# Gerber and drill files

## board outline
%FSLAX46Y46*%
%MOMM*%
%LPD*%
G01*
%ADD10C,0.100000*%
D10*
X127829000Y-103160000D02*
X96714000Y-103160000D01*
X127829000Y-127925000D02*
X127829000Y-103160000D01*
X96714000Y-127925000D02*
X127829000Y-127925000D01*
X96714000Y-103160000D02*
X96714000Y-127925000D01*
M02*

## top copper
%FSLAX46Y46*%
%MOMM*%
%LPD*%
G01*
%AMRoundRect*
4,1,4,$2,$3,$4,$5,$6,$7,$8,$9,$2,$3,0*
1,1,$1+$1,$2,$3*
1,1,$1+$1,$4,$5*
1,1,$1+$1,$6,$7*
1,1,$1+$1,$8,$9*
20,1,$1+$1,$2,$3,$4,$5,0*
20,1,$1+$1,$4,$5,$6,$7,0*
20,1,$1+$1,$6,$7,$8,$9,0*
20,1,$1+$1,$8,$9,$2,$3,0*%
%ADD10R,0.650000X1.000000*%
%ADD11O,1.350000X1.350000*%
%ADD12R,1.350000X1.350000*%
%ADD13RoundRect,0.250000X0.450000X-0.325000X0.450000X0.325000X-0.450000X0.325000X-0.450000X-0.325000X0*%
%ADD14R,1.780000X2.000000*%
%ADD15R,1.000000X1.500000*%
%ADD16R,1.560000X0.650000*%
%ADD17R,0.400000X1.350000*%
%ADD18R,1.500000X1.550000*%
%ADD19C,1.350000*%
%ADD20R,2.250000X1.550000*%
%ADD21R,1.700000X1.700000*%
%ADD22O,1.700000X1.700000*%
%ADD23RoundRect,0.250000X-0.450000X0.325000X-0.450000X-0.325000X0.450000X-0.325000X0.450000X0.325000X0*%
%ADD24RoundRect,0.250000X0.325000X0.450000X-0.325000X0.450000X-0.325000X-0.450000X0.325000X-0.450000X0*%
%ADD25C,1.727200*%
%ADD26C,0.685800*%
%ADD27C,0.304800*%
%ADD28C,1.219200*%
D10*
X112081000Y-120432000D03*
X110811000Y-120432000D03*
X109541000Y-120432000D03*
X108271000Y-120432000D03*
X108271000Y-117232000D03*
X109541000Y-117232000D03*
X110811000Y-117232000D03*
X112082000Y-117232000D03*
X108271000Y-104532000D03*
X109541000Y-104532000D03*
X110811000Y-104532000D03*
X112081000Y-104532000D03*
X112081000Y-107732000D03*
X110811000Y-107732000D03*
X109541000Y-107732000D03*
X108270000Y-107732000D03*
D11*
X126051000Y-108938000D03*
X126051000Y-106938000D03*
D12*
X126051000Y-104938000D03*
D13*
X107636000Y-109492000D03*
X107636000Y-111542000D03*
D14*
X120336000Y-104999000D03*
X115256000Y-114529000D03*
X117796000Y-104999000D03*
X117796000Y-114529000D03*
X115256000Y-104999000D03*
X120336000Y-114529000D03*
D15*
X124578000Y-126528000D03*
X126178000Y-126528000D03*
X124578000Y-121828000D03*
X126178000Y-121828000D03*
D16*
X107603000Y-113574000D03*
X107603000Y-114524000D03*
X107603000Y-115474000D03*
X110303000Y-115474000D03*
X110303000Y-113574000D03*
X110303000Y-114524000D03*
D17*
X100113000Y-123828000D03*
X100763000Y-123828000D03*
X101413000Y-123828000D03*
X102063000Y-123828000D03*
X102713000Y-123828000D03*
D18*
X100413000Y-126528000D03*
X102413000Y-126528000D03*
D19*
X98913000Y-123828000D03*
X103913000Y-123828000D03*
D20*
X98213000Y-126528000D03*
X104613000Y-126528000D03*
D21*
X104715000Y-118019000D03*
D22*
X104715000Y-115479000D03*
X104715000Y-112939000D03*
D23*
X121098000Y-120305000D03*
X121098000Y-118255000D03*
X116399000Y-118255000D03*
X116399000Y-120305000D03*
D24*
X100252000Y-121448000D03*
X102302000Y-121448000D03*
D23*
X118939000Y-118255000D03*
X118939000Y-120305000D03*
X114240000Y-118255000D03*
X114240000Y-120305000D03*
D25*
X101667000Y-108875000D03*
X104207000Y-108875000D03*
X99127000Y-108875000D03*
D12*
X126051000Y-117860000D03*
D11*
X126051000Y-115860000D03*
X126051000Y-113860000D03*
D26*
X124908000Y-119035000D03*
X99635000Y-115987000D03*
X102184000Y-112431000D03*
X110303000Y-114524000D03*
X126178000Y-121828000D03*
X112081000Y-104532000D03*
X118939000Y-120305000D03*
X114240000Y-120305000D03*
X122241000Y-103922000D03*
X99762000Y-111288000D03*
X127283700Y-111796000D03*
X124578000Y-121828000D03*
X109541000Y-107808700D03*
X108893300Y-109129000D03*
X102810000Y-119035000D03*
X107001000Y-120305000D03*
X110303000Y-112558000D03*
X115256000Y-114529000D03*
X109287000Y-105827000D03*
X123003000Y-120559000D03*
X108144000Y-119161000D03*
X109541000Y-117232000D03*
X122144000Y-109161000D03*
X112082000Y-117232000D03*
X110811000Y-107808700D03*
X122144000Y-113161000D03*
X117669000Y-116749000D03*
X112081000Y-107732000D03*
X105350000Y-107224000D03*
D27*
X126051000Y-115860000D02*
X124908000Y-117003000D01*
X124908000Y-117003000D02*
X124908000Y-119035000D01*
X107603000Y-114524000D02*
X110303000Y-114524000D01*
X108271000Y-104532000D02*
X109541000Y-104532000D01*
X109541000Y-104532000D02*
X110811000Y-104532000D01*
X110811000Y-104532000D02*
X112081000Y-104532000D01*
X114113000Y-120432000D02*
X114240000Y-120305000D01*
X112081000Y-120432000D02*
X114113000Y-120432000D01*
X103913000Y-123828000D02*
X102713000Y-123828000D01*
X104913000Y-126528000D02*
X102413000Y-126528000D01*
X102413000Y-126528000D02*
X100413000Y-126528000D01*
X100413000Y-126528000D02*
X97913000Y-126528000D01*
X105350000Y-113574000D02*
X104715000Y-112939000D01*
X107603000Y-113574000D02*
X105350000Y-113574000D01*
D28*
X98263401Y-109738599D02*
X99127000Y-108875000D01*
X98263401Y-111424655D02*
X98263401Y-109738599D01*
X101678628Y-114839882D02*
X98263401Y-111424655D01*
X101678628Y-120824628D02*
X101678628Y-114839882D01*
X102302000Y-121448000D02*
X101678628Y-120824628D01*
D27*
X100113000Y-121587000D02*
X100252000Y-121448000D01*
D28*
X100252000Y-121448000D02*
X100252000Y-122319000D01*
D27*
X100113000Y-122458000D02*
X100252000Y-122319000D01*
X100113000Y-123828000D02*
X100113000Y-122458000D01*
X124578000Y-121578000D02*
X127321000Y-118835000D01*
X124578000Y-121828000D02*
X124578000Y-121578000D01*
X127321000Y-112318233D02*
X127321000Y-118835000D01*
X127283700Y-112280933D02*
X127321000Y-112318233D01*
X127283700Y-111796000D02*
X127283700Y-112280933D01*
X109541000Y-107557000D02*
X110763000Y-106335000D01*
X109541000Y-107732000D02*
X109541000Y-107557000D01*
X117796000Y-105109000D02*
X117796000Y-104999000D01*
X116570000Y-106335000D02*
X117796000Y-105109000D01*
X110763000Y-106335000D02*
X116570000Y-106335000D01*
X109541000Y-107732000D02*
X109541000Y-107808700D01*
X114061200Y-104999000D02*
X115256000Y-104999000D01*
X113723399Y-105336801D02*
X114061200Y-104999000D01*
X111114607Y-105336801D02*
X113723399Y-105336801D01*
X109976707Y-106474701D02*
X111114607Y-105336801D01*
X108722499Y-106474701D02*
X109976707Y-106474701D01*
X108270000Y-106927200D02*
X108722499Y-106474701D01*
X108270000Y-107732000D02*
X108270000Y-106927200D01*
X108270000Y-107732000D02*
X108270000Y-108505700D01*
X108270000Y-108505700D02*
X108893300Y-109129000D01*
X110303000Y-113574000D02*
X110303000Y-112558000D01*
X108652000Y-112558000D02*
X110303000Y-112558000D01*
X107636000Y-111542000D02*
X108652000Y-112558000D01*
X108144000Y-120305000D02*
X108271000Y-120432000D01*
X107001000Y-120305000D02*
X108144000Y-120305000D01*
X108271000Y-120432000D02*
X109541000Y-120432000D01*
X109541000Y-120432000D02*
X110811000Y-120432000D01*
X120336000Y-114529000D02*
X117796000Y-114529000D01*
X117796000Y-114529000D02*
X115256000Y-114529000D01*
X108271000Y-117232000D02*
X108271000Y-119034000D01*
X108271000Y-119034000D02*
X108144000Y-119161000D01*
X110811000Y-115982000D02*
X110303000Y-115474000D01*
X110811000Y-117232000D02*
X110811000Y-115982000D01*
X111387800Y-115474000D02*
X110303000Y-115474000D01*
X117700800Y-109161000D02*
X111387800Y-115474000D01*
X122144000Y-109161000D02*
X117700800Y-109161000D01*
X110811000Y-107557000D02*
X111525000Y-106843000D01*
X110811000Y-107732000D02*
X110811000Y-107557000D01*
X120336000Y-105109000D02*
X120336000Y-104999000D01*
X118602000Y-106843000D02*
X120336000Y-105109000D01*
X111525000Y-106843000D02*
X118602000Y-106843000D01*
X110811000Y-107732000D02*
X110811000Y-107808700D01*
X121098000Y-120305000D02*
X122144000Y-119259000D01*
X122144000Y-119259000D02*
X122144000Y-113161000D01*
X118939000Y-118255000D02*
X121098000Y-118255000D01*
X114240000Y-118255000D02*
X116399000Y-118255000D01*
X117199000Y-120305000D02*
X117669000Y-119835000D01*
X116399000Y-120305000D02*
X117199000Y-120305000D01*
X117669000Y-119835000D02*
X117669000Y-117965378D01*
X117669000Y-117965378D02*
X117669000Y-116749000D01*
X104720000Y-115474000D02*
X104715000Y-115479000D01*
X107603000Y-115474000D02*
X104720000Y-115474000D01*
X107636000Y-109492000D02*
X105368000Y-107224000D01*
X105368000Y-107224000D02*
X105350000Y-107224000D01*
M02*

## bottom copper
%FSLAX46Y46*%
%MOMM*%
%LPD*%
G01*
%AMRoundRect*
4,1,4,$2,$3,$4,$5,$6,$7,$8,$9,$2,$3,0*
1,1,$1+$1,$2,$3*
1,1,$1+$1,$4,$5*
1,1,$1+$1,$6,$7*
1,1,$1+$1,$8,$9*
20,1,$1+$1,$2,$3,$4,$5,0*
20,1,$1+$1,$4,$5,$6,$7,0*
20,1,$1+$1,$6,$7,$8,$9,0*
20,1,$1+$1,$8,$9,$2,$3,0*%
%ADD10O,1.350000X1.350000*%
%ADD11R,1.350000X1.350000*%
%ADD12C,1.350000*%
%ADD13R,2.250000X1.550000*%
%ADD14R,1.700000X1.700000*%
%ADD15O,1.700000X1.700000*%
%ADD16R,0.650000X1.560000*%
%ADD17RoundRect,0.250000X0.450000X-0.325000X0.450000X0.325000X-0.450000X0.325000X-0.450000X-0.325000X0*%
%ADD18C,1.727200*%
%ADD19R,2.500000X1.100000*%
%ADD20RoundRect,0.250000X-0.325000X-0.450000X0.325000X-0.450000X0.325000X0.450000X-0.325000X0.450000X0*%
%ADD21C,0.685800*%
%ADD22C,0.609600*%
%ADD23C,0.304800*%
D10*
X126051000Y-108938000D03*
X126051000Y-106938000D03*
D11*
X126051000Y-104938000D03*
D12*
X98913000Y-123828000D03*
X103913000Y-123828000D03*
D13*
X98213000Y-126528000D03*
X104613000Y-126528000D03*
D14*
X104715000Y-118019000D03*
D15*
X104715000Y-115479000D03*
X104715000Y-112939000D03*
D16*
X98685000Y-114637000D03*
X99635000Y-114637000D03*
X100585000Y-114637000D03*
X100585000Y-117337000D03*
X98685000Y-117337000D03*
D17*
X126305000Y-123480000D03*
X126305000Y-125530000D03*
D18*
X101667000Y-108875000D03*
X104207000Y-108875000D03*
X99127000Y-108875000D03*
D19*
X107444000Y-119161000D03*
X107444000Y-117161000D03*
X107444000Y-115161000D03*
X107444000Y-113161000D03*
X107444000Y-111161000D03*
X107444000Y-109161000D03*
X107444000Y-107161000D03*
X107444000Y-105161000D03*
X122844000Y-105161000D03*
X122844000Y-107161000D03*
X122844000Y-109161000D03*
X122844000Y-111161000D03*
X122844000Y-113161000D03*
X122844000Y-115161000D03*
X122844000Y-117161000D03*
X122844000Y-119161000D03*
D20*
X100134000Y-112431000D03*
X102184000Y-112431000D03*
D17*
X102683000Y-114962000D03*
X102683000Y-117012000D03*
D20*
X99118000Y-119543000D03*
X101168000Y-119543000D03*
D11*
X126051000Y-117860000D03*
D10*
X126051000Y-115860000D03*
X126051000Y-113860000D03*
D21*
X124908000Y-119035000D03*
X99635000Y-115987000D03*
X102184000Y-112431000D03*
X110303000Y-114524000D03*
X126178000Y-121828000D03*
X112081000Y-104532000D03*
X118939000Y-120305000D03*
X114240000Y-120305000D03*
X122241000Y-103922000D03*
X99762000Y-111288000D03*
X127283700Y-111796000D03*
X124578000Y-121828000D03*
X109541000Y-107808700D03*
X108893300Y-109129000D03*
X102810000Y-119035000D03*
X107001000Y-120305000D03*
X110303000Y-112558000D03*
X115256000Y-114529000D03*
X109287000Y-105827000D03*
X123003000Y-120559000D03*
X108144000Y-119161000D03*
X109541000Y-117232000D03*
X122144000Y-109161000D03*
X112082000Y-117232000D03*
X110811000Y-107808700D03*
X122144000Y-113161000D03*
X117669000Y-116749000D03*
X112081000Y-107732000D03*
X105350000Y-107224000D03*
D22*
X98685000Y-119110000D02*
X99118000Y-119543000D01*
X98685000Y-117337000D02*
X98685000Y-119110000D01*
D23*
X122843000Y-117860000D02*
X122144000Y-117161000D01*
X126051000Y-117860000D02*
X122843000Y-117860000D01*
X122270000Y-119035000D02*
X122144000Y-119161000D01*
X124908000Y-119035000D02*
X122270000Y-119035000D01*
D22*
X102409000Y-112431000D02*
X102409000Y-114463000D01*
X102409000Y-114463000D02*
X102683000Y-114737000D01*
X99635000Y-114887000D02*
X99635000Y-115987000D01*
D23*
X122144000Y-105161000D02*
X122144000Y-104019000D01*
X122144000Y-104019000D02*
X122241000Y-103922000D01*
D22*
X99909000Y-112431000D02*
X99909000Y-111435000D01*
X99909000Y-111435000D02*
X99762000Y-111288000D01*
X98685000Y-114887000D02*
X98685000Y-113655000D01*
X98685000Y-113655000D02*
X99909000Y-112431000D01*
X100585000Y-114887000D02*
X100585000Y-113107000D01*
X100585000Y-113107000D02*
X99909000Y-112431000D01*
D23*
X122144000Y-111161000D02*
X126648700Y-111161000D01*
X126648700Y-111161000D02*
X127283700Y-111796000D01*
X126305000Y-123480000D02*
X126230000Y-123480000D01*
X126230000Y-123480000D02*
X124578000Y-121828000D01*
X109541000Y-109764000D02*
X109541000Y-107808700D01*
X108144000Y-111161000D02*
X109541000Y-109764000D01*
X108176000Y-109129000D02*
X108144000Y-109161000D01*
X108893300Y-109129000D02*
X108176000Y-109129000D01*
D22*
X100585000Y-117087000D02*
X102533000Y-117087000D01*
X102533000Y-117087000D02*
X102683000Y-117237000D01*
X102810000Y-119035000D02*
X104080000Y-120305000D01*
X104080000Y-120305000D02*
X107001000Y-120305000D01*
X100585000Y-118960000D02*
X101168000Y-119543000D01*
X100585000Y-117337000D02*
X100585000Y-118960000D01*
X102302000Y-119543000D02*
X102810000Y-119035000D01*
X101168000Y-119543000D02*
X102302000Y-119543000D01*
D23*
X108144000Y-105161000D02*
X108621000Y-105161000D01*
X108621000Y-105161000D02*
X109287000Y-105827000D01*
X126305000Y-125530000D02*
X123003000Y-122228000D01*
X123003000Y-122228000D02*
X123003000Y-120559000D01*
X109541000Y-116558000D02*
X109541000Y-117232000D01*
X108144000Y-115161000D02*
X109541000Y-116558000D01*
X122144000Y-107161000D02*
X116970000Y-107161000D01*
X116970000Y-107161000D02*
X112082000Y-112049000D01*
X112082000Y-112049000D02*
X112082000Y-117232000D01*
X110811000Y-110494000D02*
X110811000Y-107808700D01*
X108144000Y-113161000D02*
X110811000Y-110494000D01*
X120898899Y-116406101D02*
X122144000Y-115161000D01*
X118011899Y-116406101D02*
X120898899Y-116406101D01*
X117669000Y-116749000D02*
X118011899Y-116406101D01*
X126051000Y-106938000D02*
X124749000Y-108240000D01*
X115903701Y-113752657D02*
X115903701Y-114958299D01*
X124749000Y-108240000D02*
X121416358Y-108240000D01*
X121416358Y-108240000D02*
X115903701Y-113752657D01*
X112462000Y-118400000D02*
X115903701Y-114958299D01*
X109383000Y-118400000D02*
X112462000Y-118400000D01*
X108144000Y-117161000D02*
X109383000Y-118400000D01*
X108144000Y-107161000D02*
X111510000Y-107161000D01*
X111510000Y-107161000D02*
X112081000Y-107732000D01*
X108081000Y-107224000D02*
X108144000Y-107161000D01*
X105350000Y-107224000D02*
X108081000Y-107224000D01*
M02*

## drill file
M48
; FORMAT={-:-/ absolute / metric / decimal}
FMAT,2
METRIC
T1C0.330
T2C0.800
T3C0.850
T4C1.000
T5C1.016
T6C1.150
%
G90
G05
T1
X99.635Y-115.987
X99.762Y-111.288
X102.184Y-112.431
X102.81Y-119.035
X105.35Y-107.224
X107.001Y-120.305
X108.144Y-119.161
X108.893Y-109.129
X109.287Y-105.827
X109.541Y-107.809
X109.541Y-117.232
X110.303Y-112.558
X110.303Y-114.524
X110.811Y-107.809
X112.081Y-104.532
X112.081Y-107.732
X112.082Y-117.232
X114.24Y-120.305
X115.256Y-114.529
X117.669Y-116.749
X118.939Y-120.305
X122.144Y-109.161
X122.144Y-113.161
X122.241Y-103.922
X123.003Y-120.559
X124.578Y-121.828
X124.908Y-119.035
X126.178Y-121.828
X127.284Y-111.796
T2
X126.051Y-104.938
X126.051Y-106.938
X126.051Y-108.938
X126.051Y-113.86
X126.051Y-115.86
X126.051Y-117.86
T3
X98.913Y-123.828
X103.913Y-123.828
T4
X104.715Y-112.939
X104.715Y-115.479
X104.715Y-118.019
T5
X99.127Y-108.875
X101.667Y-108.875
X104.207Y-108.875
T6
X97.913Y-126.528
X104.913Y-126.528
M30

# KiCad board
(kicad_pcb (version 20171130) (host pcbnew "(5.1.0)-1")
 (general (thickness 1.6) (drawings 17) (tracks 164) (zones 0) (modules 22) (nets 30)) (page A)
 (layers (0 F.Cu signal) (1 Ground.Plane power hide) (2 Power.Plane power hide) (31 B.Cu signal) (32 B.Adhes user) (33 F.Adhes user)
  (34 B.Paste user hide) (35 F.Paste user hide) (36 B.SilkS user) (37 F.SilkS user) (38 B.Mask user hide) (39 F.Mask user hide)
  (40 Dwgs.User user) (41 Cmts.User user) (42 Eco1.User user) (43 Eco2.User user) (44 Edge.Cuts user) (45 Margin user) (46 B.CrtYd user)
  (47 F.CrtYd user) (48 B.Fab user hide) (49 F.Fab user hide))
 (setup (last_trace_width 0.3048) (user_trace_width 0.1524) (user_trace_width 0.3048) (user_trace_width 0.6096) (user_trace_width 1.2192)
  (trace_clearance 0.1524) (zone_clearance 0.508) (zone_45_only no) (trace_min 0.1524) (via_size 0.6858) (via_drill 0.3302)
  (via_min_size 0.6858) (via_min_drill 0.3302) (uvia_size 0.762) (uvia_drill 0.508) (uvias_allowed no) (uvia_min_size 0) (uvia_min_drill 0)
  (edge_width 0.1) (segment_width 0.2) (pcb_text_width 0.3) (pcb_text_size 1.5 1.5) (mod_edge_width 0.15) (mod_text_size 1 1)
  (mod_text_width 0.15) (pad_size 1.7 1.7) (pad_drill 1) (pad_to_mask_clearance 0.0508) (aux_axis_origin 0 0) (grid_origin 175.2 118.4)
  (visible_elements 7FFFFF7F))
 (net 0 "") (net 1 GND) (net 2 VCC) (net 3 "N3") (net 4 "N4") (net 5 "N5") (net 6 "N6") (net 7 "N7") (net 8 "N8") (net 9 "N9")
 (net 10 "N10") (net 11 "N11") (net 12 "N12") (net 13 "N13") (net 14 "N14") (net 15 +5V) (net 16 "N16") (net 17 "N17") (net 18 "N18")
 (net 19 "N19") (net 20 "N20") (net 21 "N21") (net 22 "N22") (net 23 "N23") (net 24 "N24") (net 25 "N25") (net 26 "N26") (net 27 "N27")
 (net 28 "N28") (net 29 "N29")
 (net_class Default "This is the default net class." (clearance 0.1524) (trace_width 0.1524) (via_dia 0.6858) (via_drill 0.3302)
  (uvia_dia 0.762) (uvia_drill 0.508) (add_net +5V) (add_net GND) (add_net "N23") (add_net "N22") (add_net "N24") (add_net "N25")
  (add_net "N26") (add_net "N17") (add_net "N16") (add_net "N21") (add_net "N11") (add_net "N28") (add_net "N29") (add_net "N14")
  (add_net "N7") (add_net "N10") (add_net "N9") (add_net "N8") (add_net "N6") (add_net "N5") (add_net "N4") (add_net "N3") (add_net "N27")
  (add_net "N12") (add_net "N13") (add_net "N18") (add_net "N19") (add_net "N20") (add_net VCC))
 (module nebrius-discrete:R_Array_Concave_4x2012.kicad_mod (layer F.Cu) (at 110.176 118.832 180)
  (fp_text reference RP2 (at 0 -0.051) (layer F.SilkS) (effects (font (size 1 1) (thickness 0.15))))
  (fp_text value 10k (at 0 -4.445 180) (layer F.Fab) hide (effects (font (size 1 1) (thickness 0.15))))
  (pad 8 smd rect (at -1.905 -1.6 180) (size 0.65 1) (layers F.Cu F.Paste F.Mask) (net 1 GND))
  (pad 7 smd rect (at -0.635 -1.6 180) (size 0.65 1) (layers F.Cu F.Paste F.Mask) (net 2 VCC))
  (pad 6 smd rect (at 0.635 -1.6 180) (size 0.65 1) (layers F.Cu F.Paste F.Mask) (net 2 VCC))
  (pad 5 smd rect (at 1.905 -1.6 180) (size 0.65 1) (layers F.Cu F.Paste F.Mask) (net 2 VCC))
  (pad 4 smd rect (at 1.905 1.6 180) (size 0.65 1) (layers F.Cu F.Paste F.Mask) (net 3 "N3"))
  (pad 3 smd rect (at 0.635 1.6 180) (size 0.65 1) (layers F.Cu F.Paste F.Mask) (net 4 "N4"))
  (pad 2 smd rect (at -0.635 1.6 180) (size 0.65 1) (layers F.Cu F.Paste F.Mask) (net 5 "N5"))
  (pad 1 smd rect (at -1.906 1.6 180) (size 0.65 1) (layers F.Cu F.Paste F.Mask) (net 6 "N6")))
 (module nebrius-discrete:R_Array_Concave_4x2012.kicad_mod (layer F.Cu) (at 110.176 106.132)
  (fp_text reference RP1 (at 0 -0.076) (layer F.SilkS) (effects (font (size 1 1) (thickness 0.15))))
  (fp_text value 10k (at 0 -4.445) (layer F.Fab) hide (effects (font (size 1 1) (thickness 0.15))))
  (pad 8 smd rect (at -1.905 -1.6) (size 0.65 1) (layers F.Cu F.Paste F.Mask) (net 1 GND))
  (pad 7 smd rect (at -0.635 -1.6) (size 0.65 1) (layers F.Cu F.Paste F.Mask) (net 1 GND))
  (pad 6 smd rect (at 0.635 -1.6) (size 0.65 1) (layers F.Cu F.Paste F.Mask) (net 1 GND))
  (pad 5 smd rect (at 1.905 -1.6) (size 0.65 1) (layers F.Cu F.Paste F.Mask) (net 1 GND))
  (pad 4 smd rect (at 1.905 1.6) (size 0.65 1) (layers F.Cu F.Paste F.Mask) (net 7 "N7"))
  (pad 3 smd rect (at 0.635 1.6) (size 0.65 1) (layers F.Cu F.Paste F.Mask) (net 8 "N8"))
  (pad 2 smd rect (at -0.635 1.6) (size 0.65 1) (layers F.Cu F.Paste F.Mask) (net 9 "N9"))
  (pad 1 smd rect (at -1.906 1.6) (size 0.65 1) (layers F.Cu F.Paste F.Mask) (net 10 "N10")))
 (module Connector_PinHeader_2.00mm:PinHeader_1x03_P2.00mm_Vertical (layer F.Cu) (at 126.051 104.938)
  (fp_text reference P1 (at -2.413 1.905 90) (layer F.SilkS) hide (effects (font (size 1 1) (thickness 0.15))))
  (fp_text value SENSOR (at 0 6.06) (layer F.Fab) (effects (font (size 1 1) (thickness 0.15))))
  (pad 3 thru_hole oval (at 0 4) (size 1.35 1.35) (drill 0.8) (layers *.Cu *.Mask) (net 1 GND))
  (pad 2 thru_hole oval (at 0 2) (size 1.35 1.35) (drill 0.8) (layers *.Cu *.Mask) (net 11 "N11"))
  (pad 1 thru_hole rect (at 0 0) (size 1.35 1.35) (drill 0.8) (layers *.Cu *.Mask) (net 2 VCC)))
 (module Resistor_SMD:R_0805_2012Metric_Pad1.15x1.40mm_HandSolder (layer F.Cu) (at 107.636 110.517 90)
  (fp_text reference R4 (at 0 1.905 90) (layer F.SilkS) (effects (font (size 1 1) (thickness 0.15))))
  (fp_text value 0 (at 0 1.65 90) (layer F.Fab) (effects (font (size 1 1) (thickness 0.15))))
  (pad 2 smd roundrect (at 1.025 0 90) (size 1.15 1.4) (layers F.Cu F.Paste F.Mask) (roundrect_rratio 0.217391) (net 7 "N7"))
  (pad 1 smd roundrect (at -1.025 0 90) (size 1.15 1.4) (layers F.Cu F.Paste F.Mask) (roundrect_rratio 0.217391) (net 2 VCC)))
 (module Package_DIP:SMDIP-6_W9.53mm (layer F.Cu) (at 117.796 109.764 270)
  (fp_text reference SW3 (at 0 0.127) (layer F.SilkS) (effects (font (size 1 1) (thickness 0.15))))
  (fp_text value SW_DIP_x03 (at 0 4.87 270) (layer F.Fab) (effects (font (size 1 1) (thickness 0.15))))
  (pad 1 smd rect (at -4.765 -2.54 270) (size 2 1.78) (layers F.Cu F.Paste F.Mask) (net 8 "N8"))
  (pad 4 smd rect (at 4.765 2.54 270) (size 2 1.78) (layers F.Cu F.Paste F.Mask) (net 2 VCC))
  (pad 2 smd rect (at -4.765 0 270) (size 2 1.78) (layers F.Cu F.Paste F.Mask) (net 9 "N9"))
  (pad 5 smd rect (at 4.765 0 270) (size 2 1.78) (layers F.Cu F.Paste F.Mask) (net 2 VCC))
  (pad 3 smd rect (at -4.765 2.54 270) (size 2 1.78) (layers F.Cu F.Paste F.Mask) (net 10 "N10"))
  (pad 6 smd rect (at 4.765 -2.54 270) (size 2 1.78) (layers F.Cu F.Paste F.Mask) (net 2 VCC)))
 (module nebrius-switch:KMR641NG (layer F.Cu) (at 125.378 124.178 90)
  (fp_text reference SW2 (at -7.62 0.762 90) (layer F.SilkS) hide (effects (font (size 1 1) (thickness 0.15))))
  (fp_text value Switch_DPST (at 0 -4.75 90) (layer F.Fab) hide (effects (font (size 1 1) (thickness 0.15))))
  (pad 1 smd rect (at -2.35 -0.8 90) (size 1.5 1) (layers F.Cu F.Paste F.Mask) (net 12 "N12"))
  (pad 2 smd rect (at -2.35 0.8 90) (size 1.5 1) (layers F.Cu F.Paste F.Mask) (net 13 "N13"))
  (pad 3 smd rect (at 2.35 -0.8 90) (size 1.5 1) (layers F.Cu F.Paste F.Mask) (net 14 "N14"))
  (pad 4 smd rect (at 2.35 0.8 90) (size 1.5 1) (layers F.Cu F.Paste F.Mask) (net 1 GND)))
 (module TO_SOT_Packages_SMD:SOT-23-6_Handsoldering (layer F.Cu) (at 108.953 114.524)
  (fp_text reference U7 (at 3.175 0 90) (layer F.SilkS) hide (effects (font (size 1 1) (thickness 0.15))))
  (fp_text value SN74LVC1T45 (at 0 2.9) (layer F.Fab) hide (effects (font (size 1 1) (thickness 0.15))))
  (pad 1 smd rect (at -1.35 -0.95) (size 1.56 0.65) (layers F.Cu F.Paste F.Mask) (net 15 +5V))
  (pad 2 smd rect (at -1.35 0) (size 1.56 0.65) (layers F.Cu F.Paste F.Mask) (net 1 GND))
  (pad 3 smd rect (at -1.35 0.95) (size 1.56 0.65) (layers F.Cu F.Paste F.Mask) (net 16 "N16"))
  (pad 4 smd rect (at 1.35 0.95) (size 1.56 0.65) (layers F.Cu F.Paste F.Mask) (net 5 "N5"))
  (pad 6 smd rect (at 1.35 -0.95) (size 1.56 0.65) (layers F.Cu F.Paste F.Mask) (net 2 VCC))
  (pad 5 smd rect (at 1.35 0) (size 1.56 0.65) (layers F.Cu F.Paste F.Mask) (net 1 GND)))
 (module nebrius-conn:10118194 (layer F.Cu) (at 101.413 126.528)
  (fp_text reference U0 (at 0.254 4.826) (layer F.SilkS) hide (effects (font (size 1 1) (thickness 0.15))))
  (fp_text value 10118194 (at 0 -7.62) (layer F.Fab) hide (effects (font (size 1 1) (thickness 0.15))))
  (pad 1 smd rect (at -1.3 -2.7) (size 0.4 1.35) (layers F.Cu F.Paste F.Mask) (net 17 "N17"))
  (pad 2 smd rect (at -0.65 -2.7) (size 0.4 1.35) (layers F.Cu F.Paste F.Mask) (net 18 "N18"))
  (pad 3 smd rect (at 0 -2.7) (size 0.4 1.35) (layers F.Cu F.Paste F.Mask) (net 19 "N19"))
  (pad 4 smd rect (at 0.65 -2.7) (size 0.4 1.35) (layers F.Cu F.Paste F.Mask) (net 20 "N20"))
  (pad 5 smd rect (at 1.3 -2.7) (size 0.4 1.35) (layers F.Cu F.Paste F.Mask) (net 1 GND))
  (pad 5 smd rect (at -1 0) (size 1.5 1.55) (layers F.Cu F.Paste F.Mask) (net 1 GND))
  (pad 5 smd rect (at 1 0) (size 1.5 1.55) (layers F.Cu F.Paste F.Mask) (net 1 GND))
  (pad 5 thru_hole circle (at -2.5 -2.7) (size 1.35 1.35) (drill 0.85) (layers *.Cu *.Mask) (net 1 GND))
  (pad 5 thru_hole circle (at 2.5 -2.7) (size 1.35 1.35) (drill 0.85) (layers *.Cu *.Mask) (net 1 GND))
  (pad 5 thru_hole rect (at -3.5 0) (size 2.25 1.55) (drill 1.15 (offset 0.3 0)) (layers *.Cu *.Mask) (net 1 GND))
  (pad 5 thru_hole rect (at 3.5 0) (size 2.25 1.55) (drill 1.15 (offset -0.3 0)) (layers *.Cu *.Mask) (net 1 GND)))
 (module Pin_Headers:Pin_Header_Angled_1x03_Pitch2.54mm (layer F.Cu) (at 104.715 118.019 180)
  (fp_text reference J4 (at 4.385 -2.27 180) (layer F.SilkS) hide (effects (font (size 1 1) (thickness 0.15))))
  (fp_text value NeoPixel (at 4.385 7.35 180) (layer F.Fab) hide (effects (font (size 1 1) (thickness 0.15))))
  (pad 1 thru_hole rect (at 0 0 180) (size 1.7 1.7) (drill 1) (layers *.Cu *.Mask) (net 1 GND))
  (pad 2 thru_hole oval (at 0 2.54 180) (size 1.7 1.7) (drill 1) (layers *.Cu *.Mask) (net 16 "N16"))
  (pad 3 thru_hole oval (at 0 5.08 180) (size 1.7 1.7) (drill 1) (layers *.Cu *.Mask) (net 15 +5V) (zone_connect 2)))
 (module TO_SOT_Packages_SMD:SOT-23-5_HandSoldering (layer B.Cu) (at 99.635 115.987 270)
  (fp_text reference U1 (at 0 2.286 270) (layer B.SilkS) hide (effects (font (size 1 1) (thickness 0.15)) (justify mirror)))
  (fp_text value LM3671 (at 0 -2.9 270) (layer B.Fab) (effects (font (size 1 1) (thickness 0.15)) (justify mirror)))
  (pad 1 smd rect (at -1.35 0.95 270) (size 1.56 0.65) (layers B.Cu B.Paste B.Mask) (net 15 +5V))
  (pad 2 smd rect (at -1.35 0 270) (size 1.56 0.65) (layers B.Cu B.Paste B.Mask) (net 1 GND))
  (pad 3 smd rect (at -1.35 -0.95 270) (size 1.56 0.65) (layers B.Cu B.Paste B.Mask) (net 15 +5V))
  (pad 4 smd rect (at 1.35 -0.95 270) (size 1.56 0.65) (layers B.Cu B.Paste B.Mask) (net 2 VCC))
  (pad 5 smd rect (at 1.35 0.95 270) (size 1.56 0.65) (layers B.Cu B.Paste B.Mask) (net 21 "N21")))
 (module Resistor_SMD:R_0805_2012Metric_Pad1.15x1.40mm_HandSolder (layer F.Cu) (at 121.098 119.28 270)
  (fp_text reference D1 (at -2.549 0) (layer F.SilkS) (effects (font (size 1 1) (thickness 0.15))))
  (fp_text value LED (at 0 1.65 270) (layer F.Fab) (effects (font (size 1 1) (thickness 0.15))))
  (pad 2 smd roundrect (at 1.025 0 270) (size 1.15 1.4) (layers F.Cu F.Paste F.Mask) (roundrect_rratio 0.217391) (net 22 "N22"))
  (pad 1 smd roundrect (at -1.025 0 270) (size 1.15 1.4) (layers F.Cu F.Paste F.Mask) (roundrect_rratio 0.217391) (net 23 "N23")))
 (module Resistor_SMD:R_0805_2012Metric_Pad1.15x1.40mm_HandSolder (layer F.Cu) (at 116.399 119.28 270)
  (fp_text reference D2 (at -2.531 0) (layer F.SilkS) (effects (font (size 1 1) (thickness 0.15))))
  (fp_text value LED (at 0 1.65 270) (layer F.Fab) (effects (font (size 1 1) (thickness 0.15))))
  (pad 1 smd roundrect (at -1.025 0 270) (size 1.15 1.4) (layers F.Cu F.Paste F.Mask) (roundrect_rratio 0.217391) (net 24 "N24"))
  (pad 2 smd roundrect (at 1.025 0 270) (size 1.15 1.4) (layers F.Cu F.Paste F.Mask) (roundrect_rratio 0.217391) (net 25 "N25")))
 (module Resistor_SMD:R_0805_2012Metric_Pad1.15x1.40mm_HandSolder (layer F.Cu) (at 101.277 121.448 180)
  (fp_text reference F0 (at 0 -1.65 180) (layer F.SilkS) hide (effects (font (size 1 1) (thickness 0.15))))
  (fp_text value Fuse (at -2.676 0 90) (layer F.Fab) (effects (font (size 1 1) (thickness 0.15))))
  (pad 2 smd roundrect (at 1.025 0 180) (size 1.15 1.4) (layers F.Cu F.Paste F.Mask) (roundrect_rratio 0.217391) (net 17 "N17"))
  (pad 1 smd roundrect (at -1.025 0 180) (size 1.15 1.4) (layers F.Cu F.Paste F.Mask) (roundrect_rratio 0.217391) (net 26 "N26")))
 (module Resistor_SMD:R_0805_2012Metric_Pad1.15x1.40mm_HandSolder (layer B.Cu) (at 126.305 124.505 90)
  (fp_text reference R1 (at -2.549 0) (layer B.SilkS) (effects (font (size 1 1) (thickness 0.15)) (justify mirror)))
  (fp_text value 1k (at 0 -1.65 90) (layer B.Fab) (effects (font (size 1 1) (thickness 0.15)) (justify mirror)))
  (pad 2 smd roundrect (at 1.025 0 90) (size 1.15 1.4) (layers B.Cu B.Paste B.Mask) (roundrect_rratio 0.217391) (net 14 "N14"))
  (pad 1 smd roundrect (at -1.025 0 90) (size 1.15 1.4) (layers B.Cu B.Paste B.Mask) (roundrect_rratio 0.217391) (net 2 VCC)))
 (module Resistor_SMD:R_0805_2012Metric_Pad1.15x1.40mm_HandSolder (layer F.Cu) (at 118.939 119.28 270)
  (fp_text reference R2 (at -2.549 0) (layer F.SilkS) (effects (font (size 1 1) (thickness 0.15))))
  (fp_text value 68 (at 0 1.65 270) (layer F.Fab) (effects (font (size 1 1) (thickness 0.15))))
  (pad 1 smd roundrect (at -1.025 0 270) (size 1.15 1.4) (layers F.Cu F.Paste F.Mask) (roundrect_rratio 0.217391) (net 23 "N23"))
  (pad 2 smd roundrect (at 1.025 0 270) (size 1.15 1.4) (layers F.Cu F.Paste F.Mask) (roundrect_rratio 0.217391) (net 1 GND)))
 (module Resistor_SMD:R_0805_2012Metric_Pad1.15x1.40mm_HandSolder (layer F.Cu) (at 114.24 119.28 270)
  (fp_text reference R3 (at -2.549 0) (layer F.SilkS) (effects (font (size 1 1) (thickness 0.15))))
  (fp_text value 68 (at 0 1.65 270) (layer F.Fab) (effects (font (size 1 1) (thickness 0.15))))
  (pad 1 smd roundrect (at -1.025 0 270) (size 1.15 1.4) (layers F.Cu F.Paste F.Mask) (roundrect_rratio 0.217391) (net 24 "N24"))
  (pad 2 smd roundrect (at 1.025 0 270) (size 1.15 1.4) (layers F.Cu F.Paste F.Mask) (roundrect_rratio 0.217391) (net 1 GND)))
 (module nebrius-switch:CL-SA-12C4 (layer F.Cu) (at 101.667 108.875 180)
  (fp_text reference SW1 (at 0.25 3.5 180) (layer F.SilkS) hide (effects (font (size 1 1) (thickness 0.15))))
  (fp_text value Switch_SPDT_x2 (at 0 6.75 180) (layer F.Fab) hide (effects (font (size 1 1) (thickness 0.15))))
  (pad 2 thru_hole circle (at 0 0 180) (size 1.7272 1.7272) (drill 1.016) (layers *.Cu *.Mask F.SilkS) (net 15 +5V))
  (pad 1 thru_hole circle (at -2.54 0 180) (size 1.7272 1.7272) (drill 1.016) (layers *.Cu *.Mask F.SilkS) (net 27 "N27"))
  (pad 3 thru_hole circle (at 2.54 0 180) (size 1.7272 1.7272) (drill 1.016) (layers *.Cu *.Mask F.SilkS) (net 26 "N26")))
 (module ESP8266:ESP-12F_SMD (layer B.Cu) (at 108.144 119.161)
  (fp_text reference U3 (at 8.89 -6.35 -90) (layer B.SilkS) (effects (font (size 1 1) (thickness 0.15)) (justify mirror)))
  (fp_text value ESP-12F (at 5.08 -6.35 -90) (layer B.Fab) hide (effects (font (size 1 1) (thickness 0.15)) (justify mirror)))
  (pad 1 smd rect (at 0 0) (size 2.5 1.1) (drill (offset -0.7 0)) (layers B.Cu B.Paste B.Mask) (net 3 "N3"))
  (pad 2 smd rect (at 0 -2) (size 2.5 1.1) (drill (offset -0.7 0)) (layers B.Cu B.Paste B.Mask) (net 11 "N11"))
  (pad 3 smd rect (at 0 -4) (size 2.5 1.1) (drill (offset -0.7 0)) (layers B.Cu B.Paste B.Mask) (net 4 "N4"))
  (pad 4 smd rect (at 0 -6) (size 2.5 1.1) (drill (offset -0.7 0)) (layers B.Cu B.Paste B.Mask) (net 8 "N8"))
  (pad 5 smd rect (at 0 -8) (size 2.5 1.1) (drill (offset -0.7 0)) (layers B.Cu B.Paste B.Mask) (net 9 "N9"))
  (pad 6 smd rect (at 0 -10) (size 2.5 1.1) (drill (offset -0.7 0)) (layers B.Cu B.Paste B.Mask) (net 10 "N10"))
  (pad 7 smd rect (at 0 -12) (size 2.5 1.1) (drill (offset -0.7 0)) (layers B.Cu B.Paste B.Mask) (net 7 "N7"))
  (pad 8 smd rect (at 0 -14) (size 2.5 1.1) (drill (offset -0.7 0)) (layers B.Cu B.Paste B.Mask) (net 2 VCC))
  (pad 9 smd rect (at 14 -14) (size 2.5 1.1) (drill (offset 0.7 0)) (layers B.Cu B.Paste B.Mask) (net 1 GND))
  (pad 10 smd rect (at 14 -12) (size 2.5 1.1) (drill (offset 0.7 0)) (layers B.Cu B.Paste B.Mask) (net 6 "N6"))
  (pad 11 smd rect (at 14 -10) (size 2.5 1.1) (drill (offset 0.7 0)) (layers B.Cu B.Paste B.Mask) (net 5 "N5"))
  (pad 12 smd rect (at 14 -8) (size 2.5 1.1) (drill (offset 0.7 0)) (layers B.Cu B.Paste B.Mask) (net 14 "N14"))
  (pad 13 smd rect (at 14 -6) (size 2.5 1.1) (drill (offset 0.7 0)) (layers B.Cu B.Paste B.Mask) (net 22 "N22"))
  (pad 14 smd rect (at 14 -4) (size 2.5 1.1) (drill (offset 0.7 0)) (layers B.Cu B.Paste B.Mask) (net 25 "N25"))
  (pad 15 smd rect (at 14 -2) (size 2.5 1.1) (drill (offset 0.7 0)) (layers B.Cu B.Paste B.Mask) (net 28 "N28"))
  (pad 16 smd rect (at 14 0) (size 2.5 1.1) (drill (offset 0.7 0)) (layers B.Cu B.Paste B.Mask) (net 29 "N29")))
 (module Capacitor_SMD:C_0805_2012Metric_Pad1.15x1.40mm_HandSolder (layer B.Cu) (at 101.159 112.431)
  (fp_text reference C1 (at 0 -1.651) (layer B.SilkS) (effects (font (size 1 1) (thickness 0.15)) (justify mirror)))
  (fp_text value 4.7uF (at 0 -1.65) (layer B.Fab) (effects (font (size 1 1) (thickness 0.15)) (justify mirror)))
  (pad 1 smd roundrect (at -1.025 0) (size 1.15 1.4) (layers B.Cu B.Paste B.Mask) (roundrect_rratio 0.217391) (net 15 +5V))
  (pad 2 smd roundrect (at 1.025 0) (size 1.15 1.4) (layers B.Cu B.Paste B.Mask) (roundrect_rratio 0.217391) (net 1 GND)))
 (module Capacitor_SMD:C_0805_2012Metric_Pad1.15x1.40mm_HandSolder (layer B.Cu) (at 102.683 115.987 90)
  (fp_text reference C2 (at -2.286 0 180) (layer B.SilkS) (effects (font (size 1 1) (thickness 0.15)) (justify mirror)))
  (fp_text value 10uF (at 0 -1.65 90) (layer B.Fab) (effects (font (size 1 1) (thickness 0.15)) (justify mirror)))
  (pad 2 smd roundrect (at 1.025 0 90) (size 1.15 1.4) (layers B.Cu B.Paste B.Mask) (roundrect_rratio 0.217391) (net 1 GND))
  (pad 1 smd roundrect (at -1.025 0 90) (size 1.15 1.4) (layers B.Cu B.Paste B.Mask) (roundrect_rratio 0.217391) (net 2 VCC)))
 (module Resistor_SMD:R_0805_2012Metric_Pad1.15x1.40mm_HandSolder (layer B.Cu) (at 100.143 119.543)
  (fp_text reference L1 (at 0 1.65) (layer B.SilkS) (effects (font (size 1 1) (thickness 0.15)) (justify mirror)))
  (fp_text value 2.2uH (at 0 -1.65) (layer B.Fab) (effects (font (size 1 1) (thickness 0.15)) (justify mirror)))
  (pad 1 smd roundrect (at -1.025 0) (size 1.15 1.4) (layers B.Cu B.Paste B.Mask) (roundrect_rratio 0.217391) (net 21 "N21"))
  (pad 2 smd roundrect (at 1.025 0) (size 1.15 1.4) (layers B.Cu B.Paste B.Mask) (roundrect_rratio 0.217391) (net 2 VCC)))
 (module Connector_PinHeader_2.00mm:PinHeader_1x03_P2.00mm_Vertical (layer F.Cu) (at 126.051 117.86 180)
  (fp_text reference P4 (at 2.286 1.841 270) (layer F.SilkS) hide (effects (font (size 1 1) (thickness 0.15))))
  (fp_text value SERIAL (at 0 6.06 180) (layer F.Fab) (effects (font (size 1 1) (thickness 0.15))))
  (pad 1 thru_hole rect (at 0 0 180) (size 1.35 1.35) (drill 0.8) (layers *.Cu *.Mask) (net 28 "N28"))
  (pad 2 thru_hole oval (at 0 2 180) (size 1.35 1.35) (drill 0.8) (layers *.Cu *.Mask) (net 29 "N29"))
  (pad 3 thru_hole oval (at 0 4 180) (size 1.35 1.35) (drill 0.8) (layers *.Cu *.Mask) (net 1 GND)))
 (gr_line (start 127.829 103.16) (end 96.714 103.16) (angle 90) (layer Edge.Cuts) (width 0.1))
 (gr_line (start 127.829 127.925) (end 127.829 103.16) (angle 90) (layer Edge.Cuts) (width 0.1))
 (gr_line (start 96.714 127.925) (end 127.829 127.925) (angle 90) (layer Edge.Cuts) (width 0.1))
 (gr_line (start 96.714 103.16) (end 96.714 127.925) (angle 90) (layer Edge.Cuts) (width 0.1))
 (segment (start 98.685 119.11) (end 99.118 119.543) (width 0.6096) (layer B.Cu) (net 21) (status 30))
 (segment (start 98.685 117.337) (end 98.685 119.11) (width 0.6096) (layer B.Cu) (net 21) (status 30))
 (segment (start 122.843 117.86) (end 122.144 117.161) (width 0.3048) (layer B.Cu) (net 28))
 (segment (start 126.051 117.86) (end 122.843 117.86) (width 0.3048) (layer B.Cu) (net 28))
 (via (at 124.908 119.035) (size 0.6858) (drill 0.3302) (layers F.Cu B.Cu) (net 29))
 (segment (start 126.051 115.86) (end 124.908 117.003) (width 0.3048) (layer F.Cu) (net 29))
 (segment (start 124.908 117.003) (end 124.908 119.035) (width 0.3048) (layer F.Cu) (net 29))
 (segment (start 122.27 119.035) (end 122.144 119.161) (width 0.3048) (layer B.Cu) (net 29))
 (segment (start 124.908 119.035) (end 122.27 119.035) (width 0.3048) (layer B.Cu) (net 29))
 (segment (start 102.409 112.431) (end 102.409 114.463) (width 0.6096) (layer B.Cu) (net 1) (status 30))
 (segment (start 102.409 114.463) (end 102.683 114.737) (width 0.6096) (layer B.Cu) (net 1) (status 30))
 (segment (start 99.635 114.887) (end 99.635 115.987) (width 0.6096) (layer B.Cu) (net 1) (status 10))
 (via (at 99.635 115.987) (size 0.6858) (drill 0.3302) (layers F.Cu B.Cu) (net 1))
 (via (at 102.184 112.431) (size 0.6858) (drill 0.3302) (layers F.Cu B.Cu) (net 1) (status 30))
 (segment (start 107.603 114.524) (end 110.303 114.524) (width 0.3048) (layer F.Cu) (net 1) (status 30))
 (via (at 110.303 114.524) (size 0.6858) (drill 0.3302) (layers F.Cu B.Cu) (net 1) (status 30))
 (via (at 126.178 121.828) (size 0.6858) (drill 0.3302) (layers F.Cu B.Cu) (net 1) (status 30))
 (segment (start 108.271 104.532) (end 109.541 104.532) (width 0.3048) (layer F.Cu) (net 1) (status 30))
 (segment (start 109.541 104.532) (end 110.811 104.532) (width 0.3048) (layer F.Cu) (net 1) (status 30))
 (segment (start 110.811 104.532) (end 112.081 104.532) (width 0.3048) (layer F.Cu) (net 1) (status 30))
 (via (at 112.081 104.532) (size 0.6858) (drill 0.3302) (layers F.Cu B.Cu) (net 1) (status 30))
 (via (at 118.939 120.305) (size 0.6858) (drill 0.3302) (layers F.Cu B.Cu) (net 1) (status 30))
 (via (at 114.24 120.305) (size 0.6858) (drill 0.3302) (layers F.Cu B.Cu) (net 1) (status 30))
 (segment (start 114.113 120.432) (end 114.24 120.305) (width 0.3048) (layer F.Cu) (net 1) (status 30))
 (segment (start 112.081 120.432) (end 114.113 120.432) (width 0.3048) (layer F.Cu) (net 1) (status 30))
 (via (at 122.241 103.922) (size 0.6858) (drill 0.3302) (layers F.Cu B.Cu) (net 1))
 (segment (start 122.144 105.161) (end 122.144 104.019) (width 0.3048) (layer B.Cu) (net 1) (status 10))
 (segment (start 122.144 104.019) (end 122.241 103.922) (width 0.3048) (layer B.Cu) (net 1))
 (segment (start 103.913 123.828) (end 102.713 123.828) (width 0.3048) (layer F.Cu) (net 1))
 (segment (start 104.913 126.528) (end 102.413 126.528) (width 0.3048) (layer F.Cu) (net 1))
 (segment (start 102.413 126.528) (end 100.413 126.528) (width 0.3048) (layer F.Cu) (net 1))
 (segment (start 100.413 126.528) (end 97.913 126.528) (width 0.3048) (layer F.Cu) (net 1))
 (segment (start 99.909 112.431) (end 99.909 111.435) (width 0.6096) (layer B.Cu) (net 15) (status 10))
 (via (at 99.762 111.288) (size 0.6858) (drill 0.3302) (layers F.Cu B.Cu) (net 15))
 (segment (start 99.909 111.435) (end 99.762 111.288) (width 0.6096) (layer B.Cu) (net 15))
 (segment (start 98.685 114.887) (end 98.685 113.655) (width 0.6096) (layer B.Cu) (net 15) (status 10))
 (segment (start 98.685 113.655) (end 99.909 112.431) (width 0.6096) (layer B.Cu) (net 15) (status 20))
 (segment (start 100.585 114.887) (end 100.585 113.107) (width 0.6096) (layer B.Cu) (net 15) (status 10))
 (segment (start 100.585 113.107) (end 99.909 112.431) (width 0.6096) (layer B.Cu) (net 15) (status 20))
 (segment (start 105.35 113.574) (end 104.715 112.939) (width 0.3048) (layer F.Cu) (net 15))
 (segment (start 107.603 113.574) (end 105.35 113.574) (width 0.3048) (layer F.Cu) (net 15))
 (segment (start 98.263401 109.738599) (end 99.127 108.875) (width 1.2192) (layer F.Cu) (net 26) (status 20))
 (segment (start 98.263401 111.424655) (end 98.263401 109.738599) (width 1.2192) (layer F.Cu) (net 26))
 (segment (start 101.678628 114.839882) (end 98.263401 111.424655) (width 1.2192) (layer F.Cu) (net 26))
 (segment (start 101.678628 120.824628) (end 101.678628 114.839882) (width 1.2192) (layer F.Cu) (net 26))
 (segment (start 102.302 121.448) (end 101.678628 120.824628) (width 1.2192) (layer F.Cu) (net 26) (status 10))
 (segment (start 100.113 121.587) (end 100.252 121.448) (width 0.3048) (layer F.Cu) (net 17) (status 30))
 (segment (start 100.252 121.448) (end 100.252 122.319) (width 1.2192) (layer F.Cu) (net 17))
 (segment (start 100.113 122.458) (end 100.252 122.319) (width 0.3048) (layer F.Cu) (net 17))
 (segment (start 100.113 123.828) (end 100.113 122.458) (width 0.3048) (layer F.Cu) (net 17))
 (segment (start 124.578 121.578) (end 127.321 118.835) (width 0.3048) (layer F.Cu) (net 14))
 (segment (start 124.578 121.828) (end 124.578 121.578) (width 0.3048) (layer F.Cu) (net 14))
 (via (at 127.2837 111.796) (size 0.6858) (drill 0.3302) (layers F.Cu B.Cu) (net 14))
 (segment (start 122.144 111.161) (end 126.6487 111.161) (width 0.3048) (layer B.Cu) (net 14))
 (segment (start 126.6487 111.161) (end 127.2837 111.796) (width 0.3048) (layer B.Cu) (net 14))
 (segment (start 127.321 112.318233) (end 127.321 118.835) (width 0.3048) (layer F.Cu) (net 14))
 (segment (start 127.2837 112.280933) (end 127.321 112.318233) (width 0.3048) (layer F.Cu) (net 14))
 (segment (start 127.2837 111.796) (end 127.2837 112.280933) (width 0.3048) (layer F.Cu) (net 14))
 (via (at 124.578 121.828) (size 0.6858) (drill 0.3302) (layers F.Cu B.Cu) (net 14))
 (segment (start 126.305 123.48) (end 126.23 123.48) (width 0.3048) (layer B.Cu) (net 14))
 (segment (start 126.23 123.48) (end 124.578 121.828) (width 0.3048) (layer B.Cu) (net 14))
 (segment (start 109.541 107.557) (end 110.763 106.335) (width 0.3048) (layer F.Cu) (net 9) (status 10))
 (segment (start 109.541 107.732) (end 109.541 107.557) (width 0.3048) (layer F.Cu) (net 9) (status 30))
 (segment (start 117.796 105.109) (end 117.796 104.999) (width 0.3048) (layer F.Cu) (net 9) (status 30))
 (segment (start 116.57 106.335) (end 117.796 105.109) (width 0.3048) (layer F.Cu) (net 9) (status 20))
 (segment (start 110.763 106.335) (end 116.57 106.335) (width 0.3048) (layer F.Cu) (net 9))
 (via (at 109.541 107.8087) (size 0.6858) (drill 0.3302) (layers F.Cu B.Cu) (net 9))
 (segment (start 109.541 107.732) (end 109.541 107.8087) (width 0.3048) (layer F.Cu) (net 9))
 (segment (start 109.541 109.764) (end 109.541 107.8087) (width 0.3048) (layer B.Cu) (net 9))
 (segment (start 108.144 111.161) (end 109.541 109.764) (width 0.3048) (layer B.Cu) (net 9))
 (segment (start 114.0612 104.999) (end 115.256 104.999) (width 0.3048) (layer F.Cu) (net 10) (status 20))
 (segment (start 113.723399 105.336801) (end 114.0612 104.999) (width 0.3048) (layer F.Cu) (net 10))
 (segment (start 111.114607 105.336801) (end 113.723399 105.336801) (width 0.3048) (layer F.Cu) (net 10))
 (segment (start 109.976707 106.474701) (end 111.114607 105.336801) (width 0.3048) (layer F.Cu) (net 10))
 (segment (start 108.722499 106.474701) (end 109.976707 106.474701) (width 0.3048) (layer F.Cu) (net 10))
 (segment (start 108.27 106.9272) (end 108.722499 106.474701) (width 0.3048) (layer F.Cu) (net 10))
 (segment (start 108.27 107.732) (end 108.27 106.9272) (width 0.3048) (layer F.Cu) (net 10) (status 10))
 (via (at 108.8933 109.129) (size 0.6858) (drill 0.3302) (layers F.Cu B.Cu) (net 10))
 (segment (start 108.27 107.732) (end 108.27 108.5057) (width 0.3048) (layer F.Cu) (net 10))
 (segment (start 108.27 108.5057) (end 108.8933 109.129) (width 0.3048) (layer F.Cu) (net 10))
 (segment (start 108.176 109.129) (end 108.144 109.161) (width 0.3048) (layer B.Cu) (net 10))
 (segment (start 108.8933 109.129) (end 108.176 109.129) (width 0.3048) (layer B.Cu) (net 10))
 (via (at 102.81 119.035) (size 0.6858) (drill 0.3302) (layers F.Cu B.Cu) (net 2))
 (segment (start 100.585 117.087) (end 102.533 117.087) (width 0.6096) (layer B.Cu) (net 2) (status 30))
 (segment (start 102.533 117.087) (end 102.683 117.237) (width 0.6096) (layer B.Cu) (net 2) (status 30))
 (via (at 107.001 120.305) (size 0.6858) (drill 0.3302) (layers F.Cu B.Cu) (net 2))
 (segment (start 102.81 119.035) (end 104.08 120.305) (width 0.6096) (layer B.Cu) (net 2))
 (segment (start 104.08 120.305) (end 107.001 120.305) (width 0.6096) (layer B.Cu) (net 2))
 (via (at 110.303 112.558) (size 0.6858) (drill 0.3302) (layers F.Cu B.Cu) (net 2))
 (segment (start 110.303 113.574) (end 110.303 112.558) (width 0.3048) (layer F.Cu) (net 2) (status 10))
 (segment (start 108.652 112.558) (end 110.303 112.558) (width 0.3048) (layer F.Cu) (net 2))
 (segment (start 107.636 111.542) (end 108.652 112.558) (width 0.3048) (layer F.Cu) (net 2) (status 10))
 (segment (start 100.585 118.96) (end 101.168 119.543) (width 0.6096) (layer B.Cu) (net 2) (status 20))
 (segment (start 100.585 117.337) (end 100.585 118.96) (width 0.6096) (layer B.Cu) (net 2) (status 10))
 (segment (start 102.302 119.543) (end 102.81 119.035) (width 0.6096) (layer B.Cu) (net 2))
 (segment (start 101.168 119.543) (end 102.302 119.543) (width 0.6096) (layer B.Cu) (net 2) (status 10))
 (segment (start 108.144 120.305) (end 108.271 120.432) (width 0.3048) (layer F.Cu) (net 2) (status 30))
 (segment (start 107.001 120.305) (end 108.144 120.305) (width 0.3048) (layer F.Cu) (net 2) (status 20))
 (segment (start 108.271 120.432) (end 109.541 120.432) (width 0.3048) (layer F.Cu) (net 2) (status 30))
 (segment (start 109.541 120.432) (end 110.811 120.432) (width 0.3048) (layer F.Cu) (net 2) (status 30))
 (segment (start 120.336 114.529) (end 117.796 114.529) (width 0.3048) (layer F.Cu) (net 2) (status 30))
 (segment (start 117.796 114.529) (end 115.256 114.529) (width 0.3048) (layer F.Cu) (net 2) (status 30))
 (via (at 115.256 114.529) (size 0.6858) (drill 0.3302) (layers F.Cu B.Cu) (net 2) (status 30))
 (via (at 109.287 105.827) (size 0.6858) (drill 0.3302) (layers F.Cu B.Cu) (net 2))
 (segment (start 108.144 105.161) (end 108.621 105.161) (width 0.3048) (layer B.Cu) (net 2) (status 30))
 (segment (start 108.621 105.161) (end 109.287 105.827) (width 0.3048) (layer B.Cu) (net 2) (status 10))
 (via (at 123.003 120.559) (size 0.6858) (drill 0.3302) (layers F.Cu B.Cu) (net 2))
 (segment (start 126.305 125.53) (end 123.003 122.228) (width 0.3048) (layer B.Cu) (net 2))
 (segment (start 123.003 122.228) (end 123.003 120.559) (width 0.3048) (layer B.Cu) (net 2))
 (via (at 108.144 119.161) (size 0.6858) (drill 0.3302) (layers F.Cu B.Cu) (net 3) (status 30))
 (segment (start 108.271 117.232) (end 108.271 119.034) (width 0.3048) (layer F.Cu) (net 3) (status 10))
 (segment (start 108.271 119.034) (end 108.144 119.161) (width 0.3048) (layer F.Cu) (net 3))
 (via (at 109.541 117.232) (size 0.6858) (drill 0.3302) (layers F.Cu B.Cu) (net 4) (status 30))
 (segment (start 109.541 116.558) (end 109.541 117.232) (width 0.3048) (layer B.Cu) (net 4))
 (segment (start 108.144 115.161) (end 109.541 116.558) (width 0.3048) (layer B.Cu) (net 4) (status 10))
 (segment (start 110.811 115.982) (end 110.303 115.474) (width 0.3048) (layer F.Cu) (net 5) (status 20))
 (segment (start 110.811 117.232) (end 110.811 115.982) (width 0.3048) (layer F.Cu) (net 5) (status 10))
 (via (at 122.144 109.161) (size 0.6858) (drill 0.3302) (layers F.Cu B.Cu) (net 5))
 (segment (start 111.3878 115.474) (end 110.303 115.474) (width 0.3048) (layer F.Cu) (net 5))
 (segment (start 117.7008 109.161) (end 111.3878 115.474) (width 0.3048) (layer F.Cu) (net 5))
 (segment (start 122.144 109.161) (end 117.7008 109.161) (width 0.3048) (layer F.Cu) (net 5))
 (segment (start 122.144 107.161) (end 116.97 107.161) (width 0.3048) (layer B.Cu) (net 6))
 (via (at 112.082 117.232) (size 0.6858) (drill 0.3302) (layers F.Cu B.Cu) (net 6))
 (segment (start 116.97 107.161) (end 112.082 112.049) (width 0.3048) (layer B.Cu) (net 6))
 (segment (start 112.082 112.049) (end 112.082 117.232) (width 0.3048) (layer B.Cu) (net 6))
 (segment (start 110.811 107.557) (end 111.525 106.843) (width 0.3048) (layer F.Cu) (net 8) (status 10))
 (segment (start 110.811 107.732) (end 110.811 107.557) (width 0.3048) (layer F.Cu) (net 8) (status 30))
 (segment (start 120.336 105.109) (end 120.336 104.999) (width 0.3048) (layer F.Cu) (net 8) (status 30))
 (segment (start 118.602 106.843) (end 120.336 105.109) (width 0.3048) (layer F.Cu) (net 8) (status 20))
 (segment (start 111.525 106.843) (end 118.602 106.843) (width 0.3048) (layer F.Cu) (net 8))
 (segment (start 110.811 107.732) (end 110.811 107.8087) (width 0.3048) (layer F.Cu) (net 8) (status 30))
 (via (at 110.811 107.8087) (size 0.6858) (drill 0.3302) (layers F.Cu B.Cu) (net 8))
 (segment (start 110.811 110.494) (end 110.811 107.8087) (width 0.3048) (layer B.Cu) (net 8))
 (segment (start 108.144 113.161) (end 110.811 110.494) (width 0.3048) (layer B.Cu) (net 8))
 (via (at 122.144 113.161) (size 0.6858) (drill 0.3302) (layers F.Cu B.Cu) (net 22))
 (segment (start 121.098 120.305) (end 122.144 119.259) (width 0.3048) (layer F.Cu) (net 22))
 (segment (start 122.144 119.259) (end 122.144 113.161) (width 0.3048) (layer F.Cu) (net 22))
 (segment (start 118.939 118.255) (end 121.098 118.255) (width 0.3048) (layer F.Cu) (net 23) (status 30))
 (segment (start 114.24 118.255) (end 116.399 118.255) (width 0.3048) (layer F.Cu) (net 24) (status 30))
 (segment (start 117.199 120.305) (end 117.669 119.835) (width 0.3048) (layer F.Cu) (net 25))
 (segment (start 116.399 120.305) (end 117.199 120.305) (width 0.3048) (layer F.Cu) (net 25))
 (via (at 117.669 116.749) (size 0.6858) (drill 0.3302) (layers F.Cu B.Cu) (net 25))
 (segment (start 117.669 119.835) (end 117.669 117.965378) (width 0.3048) (layer F.Cu) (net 25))
 (segment (start 117.669 117.965378) (end 117.669 116.749) (width 0.3048) (layer F.Cu) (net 25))
 (segment (start 120.898899 116.406101) (end 122.144 115.161) (width 0.3048) (layer B.Cu) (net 25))
 (segment (start 118.011899 116.406101) (end 120.898899 116.406101) (width 0.3048) (layer B.Cu) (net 25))
 (segment (start 117.669 116.749) (end 118.011899 116.406101) (width 0.3048) (layer B.Cu) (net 25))
 (segment (start 104.72 115.474) (end 104.715 115.479) (width 0.3048) (layer F.Cu) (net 16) (status 30))
 (segment (start 107.603 115.474) (end 104.72 115.474) (width 0.3048) (layer F.Cu) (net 16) (status 30))
 (segment (start 126.051 106.938) (end 124.749 108.24) (width 0.3048) (layer B.Cu) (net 11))
 (segment (start 115.903701 113.752657) (end 115.903701 114.958299) (width 0.3048) (layer B.Cu) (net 11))
 (segment (start 124.749 108.24) (end 121.416358 108.24) (width 0.3048) (layer B.Cu) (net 11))
 (segment (start 121.416358 108.24) (end 115.903701 113.752657) (width 0.3048) (layer B.Cu) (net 11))
 (segment (start 112.462 118.4) (end 115.903701 114.958299) (width 0.3048) (layer B.Cu) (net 11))
 (segment (start 109.383 118.4) (end 112.462 118.4) (width 0.3048) (layer B.Cu) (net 11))
 (segment (start 108.144 117.161) (end 109.383 118.4) (width 0.3048) (layer B.Cu) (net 11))
 (via (at 112.081 107.732) (size 0.6858) (drill 0.3302) (layers F.Cu B.Cu) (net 7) (status 30))
 (segment (start 108.144 107.161) (end 111.51 107.161) (width 0.3048) (layer B.Cu) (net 7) (status 10))
 (segment (start 111.51 107.161) (end 112.081 107.732) (width 0.3048) (layer B.Cu) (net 7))
 (via (at 105.35 107.224) (size 0.6858) (drill 0.3302) (layers F.Cu B.Cu) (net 7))
 (segment (start 107.636 109.492) (end 105.368 107.224) (width 0.3048) (layer F.Cu) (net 7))
 (segment (start 105.368 107.224) (end 105.35 107.224) (width 0.3048) (layer F.Cu) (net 7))
 (segment (start 108.081 107.224) (end 108.144 107.161) (width 0.3048) (layer B.Cu) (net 7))
 (segment (start 105.35 107.224) (end 108.081 107.224) (width 0.3048) (layer B.Cu) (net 7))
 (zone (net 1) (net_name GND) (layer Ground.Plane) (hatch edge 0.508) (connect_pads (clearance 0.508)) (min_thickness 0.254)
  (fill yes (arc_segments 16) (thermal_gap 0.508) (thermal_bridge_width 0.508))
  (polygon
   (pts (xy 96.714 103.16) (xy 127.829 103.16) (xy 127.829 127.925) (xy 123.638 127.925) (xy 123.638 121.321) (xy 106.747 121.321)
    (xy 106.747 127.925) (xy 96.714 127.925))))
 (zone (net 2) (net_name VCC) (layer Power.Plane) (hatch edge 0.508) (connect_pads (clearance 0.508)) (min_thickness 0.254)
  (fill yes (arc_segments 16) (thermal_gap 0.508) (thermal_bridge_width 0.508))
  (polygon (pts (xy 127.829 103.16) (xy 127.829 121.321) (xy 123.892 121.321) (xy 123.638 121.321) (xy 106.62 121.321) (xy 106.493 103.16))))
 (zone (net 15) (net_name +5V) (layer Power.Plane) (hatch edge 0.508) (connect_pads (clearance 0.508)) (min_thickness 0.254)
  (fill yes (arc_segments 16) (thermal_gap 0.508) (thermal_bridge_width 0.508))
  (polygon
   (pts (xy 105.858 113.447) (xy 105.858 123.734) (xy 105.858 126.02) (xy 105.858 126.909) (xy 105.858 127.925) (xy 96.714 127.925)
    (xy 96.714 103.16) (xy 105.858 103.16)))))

